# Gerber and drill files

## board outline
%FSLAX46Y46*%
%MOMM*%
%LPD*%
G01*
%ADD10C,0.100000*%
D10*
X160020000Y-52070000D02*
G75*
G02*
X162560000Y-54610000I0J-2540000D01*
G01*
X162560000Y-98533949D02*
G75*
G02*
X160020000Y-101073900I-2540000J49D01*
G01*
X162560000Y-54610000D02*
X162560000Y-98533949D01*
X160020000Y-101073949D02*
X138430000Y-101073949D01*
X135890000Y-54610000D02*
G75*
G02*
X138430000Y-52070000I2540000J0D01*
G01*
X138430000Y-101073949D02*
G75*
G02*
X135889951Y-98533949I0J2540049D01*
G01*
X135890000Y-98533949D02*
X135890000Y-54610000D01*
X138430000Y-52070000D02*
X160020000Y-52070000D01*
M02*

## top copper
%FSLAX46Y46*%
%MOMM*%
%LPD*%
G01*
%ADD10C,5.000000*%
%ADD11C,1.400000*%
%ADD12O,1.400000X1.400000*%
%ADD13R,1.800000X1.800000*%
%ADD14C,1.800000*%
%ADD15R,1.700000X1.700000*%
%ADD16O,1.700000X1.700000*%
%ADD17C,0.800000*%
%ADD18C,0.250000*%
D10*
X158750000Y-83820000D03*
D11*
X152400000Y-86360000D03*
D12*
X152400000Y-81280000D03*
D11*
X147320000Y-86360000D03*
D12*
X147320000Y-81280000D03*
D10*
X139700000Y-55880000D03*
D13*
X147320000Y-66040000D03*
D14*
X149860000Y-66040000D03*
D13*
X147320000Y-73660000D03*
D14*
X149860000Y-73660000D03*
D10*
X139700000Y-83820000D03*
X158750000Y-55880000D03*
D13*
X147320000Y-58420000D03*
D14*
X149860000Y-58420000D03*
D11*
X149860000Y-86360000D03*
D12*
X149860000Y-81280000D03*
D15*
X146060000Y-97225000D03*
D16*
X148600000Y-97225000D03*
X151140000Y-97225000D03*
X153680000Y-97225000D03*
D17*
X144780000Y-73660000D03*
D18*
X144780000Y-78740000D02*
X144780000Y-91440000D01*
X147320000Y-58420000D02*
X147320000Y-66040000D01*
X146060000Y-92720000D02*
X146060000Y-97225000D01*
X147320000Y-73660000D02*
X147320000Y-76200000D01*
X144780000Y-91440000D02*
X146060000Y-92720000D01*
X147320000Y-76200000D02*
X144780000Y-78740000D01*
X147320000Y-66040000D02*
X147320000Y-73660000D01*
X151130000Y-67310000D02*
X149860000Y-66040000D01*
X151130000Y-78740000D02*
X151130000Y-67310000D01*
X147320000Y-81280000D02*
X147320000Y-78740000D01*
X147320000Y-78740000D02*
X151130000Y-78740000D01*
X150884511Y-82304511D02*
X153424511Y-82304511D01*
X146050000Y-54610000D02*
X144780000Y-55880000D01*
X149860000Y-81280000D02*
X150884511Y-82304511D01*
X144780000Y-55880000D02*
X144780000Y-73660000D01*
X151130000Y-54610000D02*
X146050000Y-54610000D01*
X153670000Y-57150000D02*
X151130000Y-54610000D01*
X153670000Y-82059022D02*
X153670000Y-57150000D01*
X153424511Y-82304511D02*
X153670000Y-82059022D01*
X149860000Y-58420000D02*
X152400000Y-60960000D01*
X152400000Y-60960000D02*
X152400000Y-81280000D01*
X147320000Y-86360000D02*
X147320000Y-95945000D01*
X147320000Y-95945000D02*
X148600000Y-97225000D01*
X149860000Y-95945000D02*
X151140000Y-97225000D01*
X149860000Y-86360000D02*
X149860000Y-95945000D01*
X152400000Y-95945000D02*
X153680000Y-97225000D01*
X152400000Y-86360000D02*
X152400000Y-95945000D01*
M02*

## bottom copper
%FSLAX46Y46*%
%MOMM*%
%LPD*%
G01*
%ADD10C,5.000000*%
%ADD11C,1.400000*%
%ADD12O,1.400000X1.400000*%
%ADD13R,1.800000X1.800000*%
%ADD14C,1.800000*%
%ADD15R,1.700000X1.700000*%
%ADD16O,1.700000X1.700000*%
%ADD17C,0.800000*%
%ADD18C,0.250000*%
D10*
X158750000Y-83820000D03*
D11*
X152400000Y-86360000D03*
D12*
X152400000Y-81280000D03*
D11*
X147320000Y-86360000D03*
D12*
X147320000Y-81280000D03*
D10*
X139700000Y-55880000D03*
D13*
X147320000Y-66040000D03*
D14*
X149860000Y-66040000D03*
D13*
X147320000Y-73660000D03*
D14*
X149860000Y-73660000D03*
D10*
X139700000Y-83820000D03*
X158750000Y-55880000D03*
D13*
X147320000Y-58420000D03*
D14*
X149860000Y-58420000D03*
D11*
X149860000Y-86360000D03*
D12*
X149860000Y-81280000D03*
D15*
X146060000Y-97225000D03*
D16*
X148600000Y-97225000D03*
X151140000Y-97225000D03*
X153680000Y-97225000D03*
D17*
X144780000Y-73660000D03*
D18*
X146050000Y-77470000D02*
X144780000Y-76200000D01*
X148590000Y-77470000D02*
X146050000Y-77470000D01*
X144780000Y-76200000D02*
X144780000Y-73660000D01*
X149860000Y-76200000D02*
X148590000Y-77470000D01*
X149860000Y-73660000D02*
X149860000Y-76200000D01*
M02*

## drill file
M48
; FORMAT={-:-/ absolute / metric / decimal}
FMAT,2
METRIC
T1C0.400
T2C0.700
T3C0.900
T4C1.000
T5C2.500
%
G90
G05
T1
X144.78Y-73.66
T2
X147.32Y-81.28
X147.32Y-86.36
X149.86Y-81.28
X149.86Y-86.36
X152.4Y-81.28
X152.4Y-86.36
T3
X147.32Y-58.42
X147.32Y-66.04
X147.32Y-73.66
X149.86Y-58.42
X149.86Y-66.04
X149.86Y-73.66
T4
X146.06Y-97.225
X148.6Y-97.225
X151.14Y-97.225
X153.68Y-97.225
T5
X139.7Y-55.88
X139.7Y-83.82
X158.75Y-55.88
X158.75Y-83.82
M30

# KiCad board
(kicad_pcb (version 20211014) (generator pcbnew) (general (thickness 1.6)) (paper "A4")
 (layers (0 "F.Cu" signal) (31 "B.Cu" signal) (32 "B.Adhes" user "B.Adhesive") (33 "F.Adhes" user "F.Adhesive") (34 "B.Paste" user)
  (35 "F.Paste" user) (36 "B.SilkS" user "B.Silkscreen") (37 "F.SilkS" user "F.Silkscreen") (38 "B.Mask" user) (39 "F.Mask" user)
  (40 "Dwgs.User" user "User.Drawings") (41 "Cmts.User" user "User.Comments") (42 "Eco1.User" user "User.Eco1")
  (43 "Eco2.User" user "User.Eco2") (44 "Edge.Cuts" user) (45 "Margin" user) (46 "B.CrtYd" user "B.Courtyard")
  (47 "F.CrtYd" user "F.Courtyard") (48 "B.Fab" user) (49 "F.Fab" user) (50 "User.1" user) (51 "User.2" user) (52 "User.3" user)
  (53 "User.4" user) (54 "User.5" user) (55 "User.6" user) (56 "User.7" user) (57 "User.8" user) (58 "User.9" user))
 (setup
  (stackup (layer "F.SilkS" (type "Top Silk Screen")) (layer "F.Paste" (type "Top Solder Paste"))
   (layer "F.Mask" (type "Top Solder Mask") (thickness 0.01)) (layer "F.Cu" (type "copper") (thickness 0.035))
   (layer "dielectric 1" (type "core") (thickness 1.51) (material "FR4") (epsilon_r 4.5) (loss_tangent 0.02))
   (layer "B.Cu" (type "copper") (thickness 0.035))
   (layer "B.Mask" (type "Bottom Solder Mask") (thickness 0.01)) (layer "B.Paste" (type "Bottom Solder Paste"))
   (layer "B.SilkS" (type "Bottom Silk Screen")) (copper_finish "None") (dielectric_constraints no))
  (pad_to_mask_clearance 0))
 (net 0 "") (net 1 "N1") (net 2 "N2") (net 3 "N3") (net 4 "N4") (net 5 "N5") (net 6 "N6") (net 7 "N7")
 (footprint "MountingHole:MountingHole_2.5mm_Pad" (layer "F.Cu") (at 158.75 83.82)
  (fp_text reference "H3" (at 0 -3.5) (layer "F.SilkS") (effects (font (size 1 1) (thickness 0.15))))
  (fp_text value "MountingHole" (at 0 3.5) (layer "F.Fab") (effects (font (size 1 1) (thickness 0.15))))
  (pad "1" thru_hole circle locked (at 0 0) (size 5 5) (drill 2.5) (layers *.Cu *.Mask)))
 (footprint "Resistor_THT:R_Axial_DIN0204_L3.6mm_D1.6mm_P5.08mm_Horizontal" (layer "F.Cu") (at 152.4 86.36 90)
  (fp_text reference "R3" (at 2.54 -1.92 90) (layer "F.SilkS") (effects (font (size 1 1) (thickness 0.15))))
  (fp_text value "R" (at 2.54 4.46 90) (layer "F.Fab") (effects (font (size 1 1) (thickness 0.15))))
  (pad "1" thru_hole circle locked (at 0 0 90) (size 1.4 1.4) (drill 0.7) (layers *.Cu *.Mask) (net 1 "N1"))
  (pad "2" thru_hole oval locked (at 5.08 0 90) (size 1.4 1.4) (drill 0.7) (layers *.Cu *.Mask) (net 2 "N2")))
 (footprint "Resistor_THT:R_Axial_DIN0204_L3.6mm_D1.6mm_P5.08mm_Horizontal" (layer "F.Cu") (at 147.32 86.36 90)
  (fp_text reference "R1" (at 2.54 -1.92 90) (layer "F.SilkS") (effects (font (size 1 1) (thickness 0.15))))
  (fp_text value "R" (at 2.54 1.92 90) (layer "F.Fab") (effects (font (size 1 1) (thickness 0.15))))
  (pad "1" thru_hole circle locked (at 0 0 90) (size 1.4 1.4) (drill 0.7) (layers *.Cu *.Mask) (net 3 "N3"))
  (pad "2" thru_hole oval locked (at 5.08 0 90) (size 1.4 1.4) (drill 0.7) (layers *.Cu *.Mask) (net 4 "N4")))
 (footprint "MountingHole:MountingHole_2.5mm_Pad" (layer "F.Cu") (at 139.7 55.88)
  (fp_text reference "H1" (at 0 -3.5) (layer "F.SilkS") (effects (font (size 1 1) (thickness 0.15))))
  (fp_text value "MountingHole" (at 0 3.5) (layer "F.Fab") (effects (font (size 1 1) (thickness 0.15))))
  (pad "1" thru_hole circle locked (at 0 0) (size 5 5) (drill 2.5) (layers *.Cu *.Mask)))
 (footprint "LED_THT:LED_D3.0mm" (layer "F.Cu") (at 147.32 66.04)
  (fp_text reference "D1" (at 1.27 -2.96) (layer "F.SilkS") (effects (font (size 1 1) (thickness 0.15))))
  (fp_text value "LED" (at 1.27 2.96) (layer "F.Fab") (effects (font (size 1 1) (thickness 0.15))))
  (pad "1" thru_hole rect locked (at 0 0) (size 1.8 1.8) (drill 0.9) (layers *.Cu *.Mask) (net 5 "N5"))
  (pad "2" thru_hole circle locked (at 2.54 0) (size 1.8 1.8) (drill 0.9) (layers *.Cu *.Mask) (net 4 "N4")))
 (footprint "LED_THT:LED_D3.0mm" (layer "F.Cu") (at 147.32 73.66)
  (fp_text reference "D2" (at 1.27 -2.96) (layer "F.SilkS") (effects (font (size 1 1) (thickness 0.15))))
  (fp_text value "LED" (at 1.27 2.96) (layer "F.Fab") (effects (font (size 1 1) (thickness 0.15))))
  (pad "1" thru_hole rect locked (at 0 0) (size 1.8 1.8) (drill 0.9) (layers *.Cu *.Mask) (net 5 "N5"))
  (pad "2" thru_hole circle locked (at 2.54 0) (size 1.8 1.8) (drill 0.9) (layers *.Cu *.Mask) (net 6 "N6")))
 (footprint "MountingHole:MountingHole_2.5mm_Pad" (layer "F.Cu") (at 139.7 83.82)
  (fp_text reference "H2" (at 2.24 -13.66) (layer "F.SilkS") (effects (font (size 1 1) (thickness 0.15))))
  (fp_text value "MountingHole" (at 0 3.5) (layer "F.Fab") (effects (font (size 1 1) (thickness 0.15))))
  (pad "1" thru_hole circle locked (at 0 0) (size 5 5) (drill 2.5) (layers *.Cu *.Mask)))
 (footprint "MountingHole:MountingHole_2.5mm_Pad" (layer "F.Cu") (at 158.75 55.88)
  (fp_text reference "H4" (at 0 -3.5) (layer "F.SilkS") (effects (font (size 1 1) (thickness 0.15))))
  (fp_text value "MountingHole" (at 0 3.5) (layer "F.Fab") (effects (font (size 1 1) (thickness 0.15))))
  (pad "1" thru_hole circle locked (at 0 0) (size 5 5) (drill 2.5) (layers *.Cu *.Mask)))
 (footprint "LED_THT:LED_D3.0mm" (layer "F.Cu") (at 147.32 58.42)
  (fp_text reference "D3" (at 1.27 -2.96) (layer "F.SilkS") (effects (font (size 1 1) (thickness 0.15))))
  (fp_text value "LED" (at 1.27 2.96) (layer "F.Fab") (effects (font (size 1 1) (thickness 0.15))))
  (pad "1" thru_hole rect locked (at 0 0) (size 1.8 1.8) (drill 0.9) (layers *.Cu *.Mask) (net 5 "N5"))
  (pad "2" thru_hole circle locked (at 2.54 0) (size 1.8 1.8) (drill 0.9) (layers *.Cu *.Mask) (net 2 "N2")))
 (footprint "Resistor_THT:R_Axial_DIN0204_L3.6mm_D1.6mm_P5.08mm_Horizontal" (layer "F.Cu") (at 149.86 86.36 90)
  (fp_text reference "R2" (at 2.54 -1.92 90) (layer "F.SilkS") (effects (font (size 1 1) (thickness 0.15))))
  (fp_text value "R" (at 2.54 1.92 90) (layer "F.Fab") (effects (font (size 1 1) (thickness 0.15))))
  (pad "1" thru_hole circle locked (at 0 0 90) (size 1.4 1.4) (drill 0.7) (layers *.Cu *.Mask) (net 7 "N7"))
  (pad "2" thru_hole oval locked (at 5.08 0 90) (size 1.4 1.4) (drill 0.7) (layers *.Cu *.Mask) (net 6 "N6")))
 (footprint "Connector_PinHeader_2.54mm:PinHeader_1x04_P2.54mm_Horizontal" (layer "B.Cu") (at 146.06 97.225 -90)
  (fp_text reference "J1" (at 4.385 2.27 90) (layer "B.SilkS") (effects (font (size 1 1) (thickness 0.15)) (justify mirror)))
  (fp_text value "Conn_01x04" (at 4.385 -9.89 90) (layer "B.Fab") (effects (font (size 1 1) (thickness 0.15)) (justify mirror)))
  (pad "1" thru_hole rect locked (at 0 0 270) (size 1.7 1.7) (drill 1) (layers *.Cu *.Mask) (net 5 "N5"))
  (pad "2" thru_hole oval locked (at 0 -2.54 270) (size 1.7 1.7) (drill 1) (layers *.Cu *.Mask) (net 3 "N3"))
  (pad "3" thru_hole oval locked (at 0 -5.08 270) (size 1.7 1.7) (drill 1) (layers *.Cu *.Mask) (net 7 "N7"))
  (pad "4" thru_hole oval locked (at 0 -7.62 270) (size 1.7 1.7) (drill 1) (layers *.Cu *.Mask) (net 1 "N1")))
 (gr_arc (start 160.02 52.07) (mid 161.816051 52.813949) (end 162.56 54.61) (layer "Edge.Cuts") (width 0.1))
 (gr_arc (start 162.56 98.533949) (mid 161.816051 100.33) (end 160.02 101.073949) (layer "Edge.Cuts") (width 0.1))
 (gr_line (start 162.56 54.61) (end 162.56 98.533949) (layer "Edge.Cuts") (width 0.1))
 (gr_line (start 160.02 101.073949) (end 138.43 101.073949) (layer "Edge.Cuts") (width 0.1))
 (gr_arc (start 135.89 54.61) (mid 136.633949 52.813949) (end 138.43 52.07) (layer "Edge.Cuts") (width 0.1))
 (gr_arc (start 138.43 101.073949) (mid 136.633949 100.33) (end 135.89 98.533949) (layer "Edge.Cuts") (width 0.1))
 (gr_line (start 135.89 98.533949) (end 135.89 54.61) (layer "Edge.Cuts") (width 0.1))
 (gr_line (start 138.43 52.07) (end 160.02 52.07) (layer "Edge.Cuts") (width 0.1))
 (segment (start 144.78 78.74) (end 144.78 91.44) (width 0.25) (layer "F.Cu") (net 5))
 (segment (start 147.32 58.42) (end 147.32 66.04) (width 0.25) (layer "F.Cu") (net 5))
 (segment (start 146.06 92.72) (end 146.06 97.225) (width 0.25) (layer "F.Cu") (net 5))
 (segment (start 147.32 73.66) (end 147.32 76.2) (width 0.25) (layer "F.Cu") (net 5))
 (segment (start 144.78 91.44) (end 146.06 92.72) (width 0.25) (layer "F.Cu") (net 5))
 (segment (start 147.32 76.2) (end 144.78 78.74) (width 0.25) (layer "F.Cu") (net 5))
 (segment (start 147.32 66.04) (end 147.32 73.66) (width 0.25) (layer "F.Cu") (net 5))
 (segment (start 151.13 67.31) (end 149.86 66.04) (width 0.25) (layer "F.Cu") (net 4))
 (segment (start 151.13 78.74) (end 151.13 67.31) (width 0.25) (layer "F.Cu") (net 4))
 (segment (start 147.32 81.28) (end 147.32 78.74) (width 0.25) (layer "F.Cu") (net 4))
 (segment (start 147.32 78.74) (end 151.13 78.74) (width 0.25) (layer "F.Cu") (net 4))
 (segment (start 150.884511 82.304511) (end 153.424511 82.304511) (width 0.25) (layer "F.Cu") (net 6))
 (segment (start 146.05 54.61) (end 144.78 55.88) (width 0.25) (layer "F.Cu") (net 6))
 (segment (start 149.86 81.28) (end 150.884511 82.304511) (width 0.25) (layer "F.Cu") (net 6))
 (segment (start 144.78 55.88) (end 144.78 73.66) (width 0.25) (layer "F.Cu") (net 6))
 (segment (start 151.13 54.61) (end 146.05 54.61) (width 0.25) (layer "F.Cu") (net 6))
 (segment (start 153.67 57.15) (end 151.13 54.61) (width 0.25) (layer "F.Cu") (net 6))
 (segment (start 153.67 82.059022) (end 153.67 57.15) (width 0.25) (layer "F.Cu") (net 6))
 (segment (start 153.424511 82.304511) (end 153.67 82.059022) (width 0.25) (layer "F.Cu") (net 6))
 (via blind (at 144.78 73.66) (size 0.8) (drill 0.4) (layers "F.Cu" "B.Cu") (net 6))
 (segment (start 146.05 77.47) (end 144.78 76.2) (width 0.25) (layer "B.Cu") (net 6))
 (segment (start 148.59 77.47) (end 146.05 77.47) (width 0.25) (layer "B.Cu") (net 6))
 (segment (start 144.78 76.2) (end 144.78 73.66) (width 0.25) (layer "B.Cu") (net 6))
 (segment (start 149.86 76.2) (end 148.59 77.47) (width 0.25) (layer "B.Cu") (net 6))
 (segment (start 149.86 73.66) (end 149.86 76.2) (width 0.25) (layer "B.Cu") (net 6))
 (segment (start 149.86 58.42) (end 152.4 60.96) (width 0.25) (layer "F.Cu") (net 2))
 (segment (start 152.4 60.96) (end 152.4 81.28) (width 0.25) (layer "F.Cu") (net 2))
 (segment (start 147.32 86.36) (end 147.32 95.945) (width 0.25) (layer "F.Cu") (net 3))
 (segment (start 147.32 95.945) (end 148.6 97.225) (width 0.25) (layer "F.Cu") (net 3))
 (segment (start 149.86 95.945) (end 151.14 97.225) (width 0.25) (layer "F.Cu") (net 7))
 (segment (start 149.86 86.36) (end 149.86 95.945) (width 0.25) (layer "F.Cu") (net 7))
 (segment (start 152.4 95.945) (end 153.68 97.225) (width 0.25) (layer "F.Cu") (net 1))
 (segment (start 152.4 86.36) (end 152.4 95.945) (width 0.25) (layer "F.Cu") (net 1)))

